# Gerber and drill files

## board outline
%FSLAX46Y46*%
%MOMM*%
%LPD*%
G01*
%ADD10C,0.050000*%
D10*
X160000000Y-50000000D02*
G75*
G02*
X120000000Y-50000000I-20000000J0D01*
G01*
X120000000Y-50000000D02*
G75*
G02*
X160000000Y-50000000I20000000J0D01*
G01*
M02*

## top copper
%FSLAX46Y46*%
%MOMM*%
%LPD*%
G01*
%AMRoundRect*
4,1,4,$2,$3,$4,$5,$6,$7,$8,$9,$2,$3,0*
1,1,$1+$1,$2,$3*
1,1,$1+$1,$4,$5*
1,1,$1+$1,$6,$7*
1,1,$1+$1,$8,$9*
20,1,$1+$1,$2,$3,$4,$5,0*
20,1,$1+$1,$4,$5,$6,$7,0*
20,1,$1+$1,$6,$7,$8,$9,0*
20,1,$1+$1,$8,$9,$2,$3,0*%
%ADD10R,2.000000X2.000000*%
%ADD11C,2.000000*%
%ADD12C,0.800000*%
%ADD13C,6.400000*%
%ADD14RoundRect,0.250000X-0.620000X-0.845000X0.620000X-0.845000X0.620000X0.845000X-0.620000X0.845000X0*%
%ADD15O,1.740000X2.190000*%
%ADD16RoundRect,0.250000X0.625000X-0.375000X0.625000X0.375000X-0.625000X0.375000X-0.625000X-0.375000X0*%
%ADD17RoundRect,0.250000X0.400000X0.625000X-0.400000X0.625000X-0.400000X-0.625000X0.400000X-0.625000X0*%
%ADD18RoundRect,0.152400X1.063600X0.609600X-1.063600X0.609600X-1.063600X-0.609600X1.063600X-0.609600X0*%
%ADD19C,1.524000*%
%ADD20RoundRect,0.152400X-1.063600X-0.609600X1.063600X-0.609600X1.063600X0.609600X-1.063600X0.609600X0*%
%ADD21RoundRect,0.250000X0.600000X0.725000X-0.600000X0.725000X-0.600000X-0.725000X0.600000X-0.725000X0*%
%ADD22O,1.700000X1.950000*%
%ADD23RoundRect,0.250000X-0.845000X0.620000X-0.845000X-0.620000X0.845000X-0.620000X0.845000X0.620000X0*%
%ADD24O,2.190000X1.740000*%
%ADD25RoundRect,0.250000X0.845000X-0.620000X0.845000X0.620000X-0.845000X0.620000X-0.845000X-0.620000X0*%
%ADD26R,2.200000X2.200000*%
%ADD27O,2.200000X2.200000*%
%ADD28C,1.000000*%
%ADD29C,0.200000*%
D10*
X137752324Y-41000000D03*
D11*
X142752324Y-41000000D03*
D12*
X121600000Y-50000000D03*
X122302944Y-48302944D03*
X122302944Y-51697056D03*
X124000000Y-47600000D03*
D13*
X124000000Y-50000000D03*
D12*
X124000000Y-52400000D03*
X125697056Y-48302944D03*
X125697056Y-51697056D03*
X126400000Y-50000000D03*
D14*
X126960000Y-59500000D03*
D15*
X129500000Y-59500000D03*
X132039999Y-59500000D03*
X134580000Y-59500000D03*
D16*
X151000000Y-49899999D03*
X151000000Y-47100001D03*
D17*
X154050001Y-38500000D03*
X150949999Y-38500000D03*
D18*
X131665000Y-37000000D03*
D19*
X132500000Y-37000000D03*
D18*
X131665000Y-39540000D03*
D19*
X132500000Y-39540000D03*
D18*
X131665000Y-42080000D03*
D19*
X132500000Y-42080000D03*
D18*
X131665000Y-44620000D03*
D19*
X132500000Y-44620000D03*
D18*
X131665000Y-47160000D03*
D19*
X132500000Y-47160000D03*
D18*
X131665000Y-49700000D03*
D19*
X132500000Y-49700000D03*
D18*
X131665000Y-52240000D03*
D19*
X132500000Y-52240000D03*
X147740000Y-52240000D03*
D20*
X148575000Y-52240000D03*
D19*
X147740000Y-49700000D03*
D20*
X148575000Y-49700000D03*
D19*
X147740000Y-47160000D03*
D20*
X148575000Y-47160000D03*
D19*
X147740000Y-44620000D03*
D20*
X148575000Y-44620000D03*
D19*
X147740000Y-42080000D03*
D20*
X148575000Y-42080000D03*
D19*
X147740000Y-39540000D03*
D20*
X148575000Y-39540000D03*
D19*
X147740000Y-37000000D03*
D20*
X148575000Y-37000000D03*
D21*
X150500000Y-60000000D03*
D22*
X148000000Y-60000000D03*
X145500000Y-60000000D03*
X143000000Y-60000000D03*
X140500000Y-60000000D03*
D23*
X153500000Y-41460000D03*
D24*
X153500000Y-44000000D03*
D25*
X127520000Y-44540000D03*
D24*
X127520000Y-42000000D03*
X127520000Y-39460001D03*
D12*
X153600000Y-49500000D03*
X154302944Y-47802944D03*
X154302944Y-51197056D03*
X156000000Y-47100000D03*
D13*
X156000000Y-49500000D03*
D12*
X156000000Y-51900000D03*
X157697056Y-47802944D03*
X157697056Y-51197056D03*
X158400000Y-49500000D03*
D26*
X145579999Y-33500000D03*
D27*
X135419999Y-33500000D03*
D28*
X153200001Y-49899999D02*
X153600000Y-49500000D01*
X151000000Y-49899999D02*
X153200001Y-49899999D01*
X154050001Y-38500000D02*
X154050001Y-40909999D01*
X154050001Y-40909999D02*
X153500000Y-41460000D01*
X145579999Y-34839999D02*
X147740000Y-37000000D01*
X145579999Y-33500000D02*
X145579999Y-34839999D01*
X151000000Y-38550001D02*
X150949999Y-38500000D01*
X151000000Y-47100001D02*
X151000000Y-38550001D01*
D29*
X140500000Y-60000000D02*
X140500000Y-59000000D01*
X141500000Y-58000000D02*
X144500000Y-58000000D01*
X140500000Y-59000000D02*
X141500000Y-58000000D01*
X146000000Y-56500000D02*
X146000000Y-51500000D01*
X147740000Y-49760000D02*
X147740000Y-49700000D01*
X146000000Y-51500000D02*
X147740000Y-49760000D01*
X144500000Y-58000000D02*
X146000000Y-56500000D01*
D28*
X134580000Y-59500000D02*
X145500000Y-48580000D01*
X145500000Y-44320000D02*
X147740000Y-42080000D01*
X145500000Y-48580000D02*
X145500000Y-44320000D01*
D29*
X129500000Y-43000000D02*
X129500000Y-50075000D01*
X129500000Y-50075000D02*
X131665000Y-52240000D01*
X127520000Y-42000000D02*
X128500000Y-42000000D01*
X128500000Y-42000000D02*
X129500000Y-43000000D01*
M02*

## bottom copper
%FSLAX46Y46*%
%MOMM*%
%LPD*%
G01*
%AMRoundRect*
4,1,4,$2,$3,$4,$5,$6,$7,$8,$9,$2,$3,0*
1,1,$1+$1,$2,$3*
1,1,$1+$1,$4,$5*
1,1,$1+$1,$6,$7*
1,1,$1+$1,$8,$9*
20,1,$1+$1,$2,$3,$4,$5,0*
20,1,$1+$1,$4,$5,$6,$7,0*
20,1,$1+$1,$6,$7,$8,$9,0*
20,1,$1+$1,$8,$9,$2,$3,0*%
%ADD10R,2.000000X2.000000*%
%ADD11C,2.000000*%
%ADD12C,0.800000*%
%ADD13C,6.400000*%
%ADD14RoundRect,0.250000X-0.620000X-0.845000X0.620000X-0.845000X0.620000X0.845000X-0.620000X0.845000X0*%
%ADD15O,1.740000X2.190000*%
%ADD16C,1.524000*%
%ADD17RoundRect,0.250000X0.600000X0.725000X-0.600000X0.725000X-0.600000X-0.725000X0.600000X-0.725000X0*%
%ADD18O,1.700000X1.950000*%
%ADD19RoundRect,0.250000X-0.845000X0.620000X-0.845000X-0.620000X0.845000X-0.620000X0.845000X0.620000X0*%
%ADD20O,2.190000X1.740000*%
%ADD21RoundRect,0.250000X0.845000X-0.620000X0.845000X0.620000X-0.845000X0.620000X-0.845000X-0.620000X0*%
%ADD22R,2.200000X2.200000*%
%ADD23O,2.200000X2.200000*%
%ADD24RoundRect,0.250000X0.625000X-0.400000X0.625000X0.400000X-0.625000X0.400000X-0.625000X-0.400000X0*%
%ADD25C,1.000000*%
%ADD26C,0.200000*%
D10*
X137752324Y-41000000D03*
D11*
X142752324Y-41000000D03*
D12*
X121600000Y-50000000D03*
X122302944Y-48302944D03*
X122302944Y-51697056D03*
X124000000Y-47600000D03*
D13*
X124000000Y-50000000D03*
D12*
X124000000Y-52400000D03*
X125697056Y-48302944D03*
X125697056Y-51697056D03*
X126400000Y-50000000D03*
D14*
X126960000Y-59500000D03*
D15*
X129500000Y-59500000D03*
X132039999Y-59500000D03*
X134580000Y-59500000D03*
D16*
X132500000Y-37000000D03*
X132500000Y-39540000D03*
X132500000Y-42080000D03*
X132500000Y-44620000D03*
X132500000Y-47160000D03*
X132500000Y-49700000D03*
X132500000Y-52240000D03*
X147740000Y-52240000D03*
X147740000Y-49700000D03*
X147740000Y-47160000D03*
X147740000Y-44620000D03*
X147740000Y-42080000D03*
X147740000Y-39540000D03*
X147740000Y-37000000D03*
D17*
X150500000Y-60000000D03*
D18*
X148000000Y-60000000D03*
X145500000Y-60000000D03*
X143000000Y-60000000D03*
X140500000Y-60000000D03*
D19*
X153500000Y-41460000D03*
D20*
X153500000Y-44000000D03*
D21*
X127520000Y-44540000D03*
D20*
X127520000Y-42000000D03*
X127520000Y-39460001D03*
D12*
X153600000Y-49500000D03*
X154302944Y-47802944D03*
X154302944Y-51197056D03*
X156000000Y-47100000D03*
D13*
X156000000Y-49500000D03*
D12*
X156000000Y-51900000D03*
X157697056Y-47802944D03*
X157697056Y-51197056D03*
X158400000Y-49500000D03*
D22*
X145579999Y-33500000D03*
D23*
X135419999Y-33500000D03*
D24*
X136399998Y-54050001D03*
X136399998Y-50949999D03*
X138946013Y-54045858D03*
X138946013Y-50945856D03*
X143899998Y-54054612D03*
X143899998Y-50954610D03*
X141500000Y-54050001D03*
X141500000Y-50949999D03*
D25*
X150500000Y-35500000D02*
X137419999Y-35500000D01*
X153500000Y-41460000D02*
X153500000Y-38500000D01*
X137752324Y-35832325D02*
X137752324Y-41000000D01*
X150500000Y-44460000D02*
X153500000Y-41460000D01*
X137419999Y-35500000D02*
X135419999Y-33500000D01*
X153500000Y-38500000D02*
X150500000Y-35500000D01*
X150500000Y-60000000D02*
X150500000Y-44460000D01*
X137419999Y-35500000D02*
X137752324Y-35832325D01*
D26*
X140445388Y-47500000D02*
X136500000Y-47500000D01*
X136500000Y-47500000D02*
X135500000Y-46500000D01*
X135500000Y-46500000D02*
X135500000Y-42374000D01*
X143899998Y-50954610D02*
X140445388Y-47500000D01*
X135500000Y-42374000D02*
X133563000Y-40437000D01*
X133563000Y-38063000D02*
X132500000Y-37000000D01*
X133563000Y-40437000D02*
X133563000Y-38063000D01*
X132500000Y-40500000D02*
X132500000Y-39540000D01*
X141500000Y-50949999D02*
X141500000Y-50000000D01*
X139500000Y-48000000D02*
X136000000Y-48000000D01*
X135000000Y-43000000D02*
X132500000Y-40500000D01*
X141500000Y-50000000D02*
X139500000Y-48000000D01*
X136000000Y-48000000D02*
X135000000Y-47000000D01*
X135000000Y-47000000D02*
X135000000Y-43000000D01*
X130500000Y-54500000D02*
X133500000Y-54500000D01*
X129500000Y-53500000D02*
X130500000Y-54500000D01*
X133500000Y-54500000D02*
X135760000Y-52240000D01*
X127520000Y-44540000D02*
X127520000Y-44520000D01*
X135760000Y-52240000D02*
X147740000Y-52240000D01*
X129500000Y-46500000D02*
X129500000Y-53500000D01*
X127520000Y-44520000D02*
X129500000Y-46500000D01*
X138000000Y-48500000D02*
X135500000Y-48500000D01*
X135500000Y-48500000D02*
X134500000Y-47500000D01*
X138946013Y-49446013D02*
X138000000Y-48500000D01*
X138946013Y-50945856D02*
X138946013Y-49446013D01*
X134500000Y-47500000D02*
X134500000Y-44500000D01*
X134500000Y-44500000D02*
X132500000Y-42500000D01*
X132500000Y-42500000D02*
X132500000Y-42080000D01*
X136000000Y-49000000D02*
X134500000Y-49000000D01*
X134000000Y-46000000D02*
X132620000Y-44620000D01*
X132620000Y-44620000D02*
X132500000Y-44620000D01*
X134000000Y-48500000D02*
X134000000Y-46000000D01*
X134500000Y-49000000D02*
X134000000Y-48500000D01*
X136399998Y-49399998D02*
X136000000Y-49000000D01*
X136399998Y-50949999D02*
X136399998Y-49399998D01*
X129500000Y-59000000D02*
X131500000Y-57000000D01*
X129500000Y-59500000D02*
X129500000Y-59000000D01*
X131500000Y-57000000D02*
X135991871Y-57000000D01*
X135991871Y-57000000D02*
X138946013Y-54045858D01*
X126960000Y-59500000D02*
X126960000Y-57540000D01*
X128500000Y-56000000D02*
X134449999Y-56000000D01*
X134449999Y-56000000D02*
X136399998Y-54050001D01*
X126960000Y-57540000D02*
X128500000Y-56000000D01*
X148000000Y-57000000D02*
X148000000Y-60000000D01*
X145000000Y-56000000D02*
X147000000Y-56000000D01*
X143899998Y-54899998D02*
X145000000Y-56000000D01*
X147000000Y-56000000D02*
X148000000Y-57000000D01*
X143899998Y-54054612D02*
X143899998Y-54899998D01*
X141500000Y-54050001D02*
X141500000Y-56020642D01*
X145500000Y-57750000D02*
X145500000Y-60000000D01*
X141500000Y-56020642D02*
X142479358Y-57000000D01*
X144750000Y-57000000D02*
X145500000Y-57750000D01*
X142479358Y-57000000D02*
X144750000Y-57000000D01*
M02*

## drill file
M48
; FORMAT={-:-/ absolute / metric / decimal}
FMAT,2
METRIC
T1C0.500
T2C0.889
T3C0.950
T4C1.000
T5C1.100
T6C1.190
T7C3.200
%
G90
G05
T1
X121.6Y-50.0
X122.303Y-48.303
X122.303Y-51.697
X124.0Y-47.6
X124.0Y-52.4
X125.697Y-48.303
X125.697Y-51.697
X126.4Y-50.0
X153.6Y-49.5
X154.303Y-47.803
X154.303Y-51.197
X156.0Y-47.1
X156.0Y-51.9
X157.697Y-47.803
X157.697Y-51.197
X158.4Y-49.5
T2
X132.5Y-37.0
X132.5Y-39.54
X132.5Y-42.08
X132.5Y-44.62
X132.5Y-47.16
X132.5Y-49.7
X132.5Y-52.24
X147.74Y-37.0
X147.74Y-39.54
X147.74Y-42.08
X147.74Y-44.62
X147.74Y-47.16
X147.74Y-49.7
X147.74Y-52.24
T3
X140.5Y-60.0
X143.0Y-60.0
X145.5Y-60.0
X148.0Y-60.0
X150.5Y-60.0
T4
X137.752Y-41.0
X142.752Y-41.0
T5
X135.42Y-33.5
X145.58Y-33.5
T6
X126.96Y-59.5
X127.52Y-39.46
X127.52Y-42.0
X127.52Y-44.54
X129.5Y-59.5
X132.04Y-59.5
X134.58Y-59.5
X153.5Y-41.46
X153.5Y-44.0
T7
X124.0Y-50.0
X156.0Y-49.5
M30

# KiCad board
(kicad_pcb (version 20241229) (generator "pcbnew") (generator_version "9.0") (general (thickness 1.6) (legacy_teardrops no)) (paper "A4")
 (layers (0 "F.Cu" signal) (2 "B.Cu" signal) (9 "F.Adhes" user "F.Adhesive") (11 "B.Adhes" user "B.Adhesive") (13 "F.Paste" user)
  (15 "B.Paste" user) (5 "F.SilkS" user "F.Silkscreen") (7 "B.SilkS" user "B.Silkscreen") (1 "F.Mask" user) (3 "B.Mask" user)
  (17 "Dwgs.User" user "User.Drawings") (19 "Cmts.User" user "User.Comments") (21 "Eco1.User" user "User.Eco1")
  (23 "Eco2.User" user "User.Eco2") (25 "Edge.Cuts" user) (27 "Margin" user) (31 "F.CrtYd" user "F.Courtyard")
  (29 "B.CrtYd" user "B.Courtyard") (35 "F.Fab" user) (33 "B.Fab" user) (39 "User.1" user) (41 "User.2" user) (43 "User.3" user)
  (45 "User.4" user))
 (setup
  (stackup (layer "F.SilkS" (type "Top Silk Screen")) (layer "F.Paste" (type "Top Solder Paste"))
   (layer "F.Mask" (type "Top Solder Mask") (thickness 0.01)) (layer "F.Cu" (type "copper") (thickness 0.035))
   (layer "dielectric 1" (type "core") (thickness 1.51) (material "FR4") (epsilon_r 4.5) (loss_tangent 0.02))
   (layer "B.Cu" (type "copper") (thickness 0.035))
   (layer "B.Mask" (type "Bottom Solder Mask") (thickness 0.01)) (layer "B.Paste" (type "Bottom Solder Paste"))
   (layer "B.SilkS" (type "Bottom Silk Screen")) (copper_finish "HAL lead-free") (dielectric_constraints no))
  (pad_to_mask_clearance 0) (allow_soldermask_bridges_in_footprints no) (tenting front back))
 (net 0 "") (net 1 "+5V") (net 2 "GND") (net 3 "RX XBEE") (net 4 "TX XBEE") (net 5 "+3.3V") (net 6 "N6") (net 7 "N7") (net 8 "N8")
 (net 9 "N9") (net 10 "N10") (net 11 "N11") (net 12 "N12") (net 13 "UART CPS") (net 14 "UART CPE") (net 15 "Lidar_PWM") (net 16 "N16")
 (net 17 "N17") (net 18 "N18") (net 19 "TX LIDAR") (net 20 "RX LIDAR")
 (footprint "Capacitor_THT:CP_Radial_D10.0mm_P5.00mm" (layer "F.Cu") (at 137.752324 41)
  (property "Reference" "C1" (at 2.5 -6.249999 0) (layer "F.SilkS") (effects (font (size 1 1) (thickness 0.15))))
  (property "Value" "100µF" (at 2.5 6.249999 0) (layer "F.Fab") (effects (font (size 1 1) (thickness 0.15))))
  (pad "1" thru_hole rect (at 0 0) (size 2 2) (drill 1) (layers "*.Cu" "*.Mask") (remove_unused_layers no) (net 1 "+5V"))
  (pad "2" thru_hole circle (at 5 0) (size 2 2) (drill 1) (layers "*.Cu" "*.Mask") (remove_unused_layers no) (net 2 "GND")))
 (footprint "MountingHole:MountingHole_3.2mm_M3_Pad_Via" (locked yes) (layer "F.Cu") (at 124 50)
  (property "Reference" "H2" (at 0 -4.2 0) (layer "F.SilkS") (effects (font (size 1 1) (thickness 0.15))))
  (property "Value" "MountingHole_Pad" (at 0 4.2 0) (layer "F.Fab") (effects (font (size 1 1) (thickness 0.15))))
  (pad "1" thru_hole circle (at -2.4 0) (size 0.8 0.8) (drill 0.5) (layers "*.Cu" "*.Mask") (remove_unused_layers no) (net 2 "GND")
   (zone_connect 2))
  (pad "1" thru_hole circle (at -1.697056 -1.697056) (size 0.8 0.8) (drill 0.5) (layers "*.Cu" "*.Mask") (remove_unused_layers no)
   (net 2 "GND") (zone_connect 2))
  (pad "1" thru_hole circle (at -1.697056 1.697056) (size 0.8 0.8) (drill 0.5) (layers "*.Cu" "*.Mask") (remove_unused_layers no)
   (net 2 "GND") (zone_connect 2))
  (pad "1" thru_hole circle (at 0 -2.4) (size 0.8 0.8) (drill 0.5) (layers "*.Cu" "*.Mask") (remove_unused_layers no) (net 2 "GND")
   (zone_connect 2))
  (pad "1" thru_hole circle (at 0 0) (size 6.4 6.4) (drill 3.2) (layers "*.Cu" "*.Mask") (remove_unused_layers no) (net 2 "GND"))
  (pad "1" thru_hole circle (at 0 2.4) (size 0.8 0.8) (drill 0.5) (layers "*.Cu" "*.Mask") (remove_unused_layers no) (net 2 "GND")
   (zone_connect 2))
  (pad "1" thru_hole circle (at 1.697056 -1.697056) (size 0.8 0.8) (drill 0.5) (layers "*.Cu" "*.Mask") (remove_unused_layers no)
   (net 2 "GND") (zone_connect 2))
  (pad "1" thru_hole circle (at 1.697056 1.697056) (size 0.8 0.8) (drill 0.5) (layers "*.Cu" "*.Mask") (remove_unused_layers no)
   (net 2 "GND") (zone_connect 2))
  (pad "1" thru_hole circle (at 2.4 0) (size 0.8 0.8) (drill 0.5) (layers "*.Cu" "*.Mask") (remove_unused_layers no) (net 2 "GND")
   (zone_connect 2)))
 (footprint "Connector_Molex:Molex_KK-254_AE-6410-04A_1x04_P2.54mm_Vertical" (layer "F.Cu") (at 126.96 59.5)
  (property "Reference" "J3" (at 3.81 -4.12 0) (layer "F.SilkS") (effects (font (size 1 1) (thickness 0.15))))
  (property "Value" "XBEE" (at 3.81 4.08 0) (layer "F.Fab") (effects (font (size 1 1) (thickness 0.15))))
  (pad "1" thru_hole roundrect (at 0 0) (size 1.74 2.19) (drill 1.19) (layers "*.Cu" "*.Mask") (remove_unused_layers no)
   (roundrect_rratio 0.143678) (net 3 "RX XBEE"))
  (pad "2" thru_hole oval (at 2.54 0) (size 1.74 2.19) (drill 1.19) (layers "*.Cu" "*.Mask") (remove_unused_layers no) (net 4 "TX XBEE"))
  (pad "3" thru_hole oval (at 5.079999 0) (size 1.74 2.19) (drill 1.19) (layers "*.Cu" "*.Mask") (remove_unused_layers no) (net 2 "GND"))
  (pad "4" thru_hole oval (at 7.62 0) (size 1.74 2.19) (drill 1.19) (layers "*.Cu" "*.Mask") (remove_unused_layers no) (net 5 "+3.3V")))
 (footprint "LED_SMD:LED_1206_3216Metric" (layer "F.Cu") (at 151 48.5 90)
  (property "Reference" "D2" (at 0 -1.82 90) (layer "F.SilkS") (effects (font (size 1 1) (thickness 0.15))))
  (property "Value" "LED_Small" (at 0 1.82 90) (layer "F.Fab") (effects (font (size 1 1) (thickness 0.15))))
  (pad "1" smd roundrect (at -1.399999 0 90) (size 1.25 1.75) (layers "F.Cu" "F.Mask" "F.Paste") (roundrect_rratio 0.2) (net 2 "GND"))
  (pad "2" smd roundrect (at 1.399999 0 90) (size 1.25 1.75) (layers "F.Cu" "F.Mask" "F.Paste") (roundrect_rratio 0.2) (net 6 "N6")))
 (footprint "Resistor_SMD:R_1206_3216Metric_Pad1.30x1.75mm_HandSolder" (layer "F.Cu") (at 152.5 38.5 180)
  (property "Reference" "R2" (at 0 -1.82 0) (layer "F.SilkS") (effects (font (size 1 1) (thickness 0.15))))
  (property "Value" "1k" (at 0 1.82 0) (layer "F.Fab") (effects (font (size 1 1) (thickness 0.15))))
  (pad "1" smd roundrect (at -1.550001 0 180) (size 1.3 1.75) (layers "F.Cu" "F.Mask" "F.Paste") (roundrect_rratio 0.192308) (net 1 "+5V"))
  (pad "2" smd roundrect (at 1.550001 0 180) (size 1.3 1.75) (layers "F.Cu" "F.Mask" "F.Paste") (roundrect_rratio 0.192308) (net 6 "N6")))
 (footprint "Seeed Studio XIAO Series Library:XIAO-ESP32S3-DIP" (layer "F.Cu") (at 140.12 44.62)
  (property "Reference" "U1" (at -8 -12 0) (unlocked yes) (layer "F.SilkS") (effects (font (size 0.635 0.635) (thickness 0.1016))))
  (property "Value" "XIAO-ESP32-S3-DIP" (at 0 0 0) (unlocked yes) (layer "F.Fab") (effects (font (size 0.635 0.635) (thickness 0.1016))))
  (pad "1" smd roundrect (at -8.455 -7.62 180) (size 2.432 1.524) (layers "F.Cu" "F.Mask") (roundrect_rratio 0.1) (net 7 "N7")
   (thermal_bridge_angle 45))
  (pad "1" thru_hole circle (at -7.62 -7.62 180) (size 1.524 1.524) (drill 0.889) (layers "*.Cu" "*.Mask") (remove_unused_layers no)
   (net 7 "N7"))
  (pad "2" smd roundrect (at -8.455 -5.08 180) (size 2.432 1.524) (layers "F.Cu" "F.Mask") (roundrect_rratio 0.1) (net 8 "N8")
   (thermal_bridge_angle 45))
  (pad "2" thru_hole circle (at -7.62 -5.08 180) (size 1.524 1.524) (drill 0.889) (layers "*.Cu" "*.Mask") (remove_unused_layers no)
   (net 8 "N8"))
  (pad "3" smd roundrect (at -8.455 -2.54 180) (size 2.432 1.524) (layers "F.Cu" "F.Mask") (roundrect_rratio 0.1) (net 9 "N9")
   (thermal_bridge_angle 45))
  (pad "3" thru_hole circle (at -7.62 -2.54 180) (size 1.524 1.524) (drill 0.889) (layers "*.Cu" "*.Mask") (remove_unused_layers no)
   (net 9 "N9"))
  (pad "4" smd roundrect (at -8.455 0 180) (size 2.432 1.524) (layers "F.Cu" "F.Mask") (roundrect_rratio 0.1) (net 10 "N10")
   (thermal_bridge_angle 45))
  (pad "4" thru_hole circle (at -7.62 0 180) (size 1.524 1.524) (drill 0.889) (layers "*.Cu" "*.Mask") (remove_unused_layers no)
   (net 10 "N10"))
  (pad "5" smd roundrect (at -8.455 2.54 180) (size 2.432 1.524) (layers "F.Cu" "F.Mask") (roundrect_rratio 0.1) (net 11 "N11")
   (thermal_bridge_angle 45))
  (pad "5" thru_hole circle (at -7.62 2.54 180) (size 1.524 1.524) (drill 0.889) (layers "*.Cu" "*.Mask") (remove_unused_layers no)
   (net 11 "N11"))
  (pad "6" smd roundrect (at -8.455 5.08 180) (size 2.432 1.524) (layers "F.Cu" "F.Mask") (roundrect_rratio 0.1) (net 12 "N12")
   (thermal_bridge_angle 45))
  (pad "6" thru_hole circle (at -7.62 5.08 180) (size 1.524 1.524) (drill 0.889) (layers "*.Cu" "*.Mask") (remove_unused_layers no)
   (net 12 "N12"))
  (pad "7" smd roundrect (at -8.455 7.62 180) (size 2.432 1.524) (layers "F.Cu" "F.Mask") (roundrect_rratio 0.1) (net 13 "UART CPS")
   (thermal_bridge_angle 45))
  (pad "7" thru_hole circle (at -7.62 7.62 180) (size 1.524 1.524) (drill 0.889) (layers "*.Cu" "*.Mask") (remove_unused_layers no)
   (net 13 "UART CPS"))
  (pad "8" thru_hole circle (at 7.62 7.62) (size 1.524 1.524) (drill 0.889) (layers "*.Cu" "*.Mask") (remove_unused_layers no)
   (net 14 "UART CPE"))
  (pad "8" smd roundrect (at 8.455 7.62) (size 2.432 1.524) (layers "F.Cu" "F.Mask") (roundrect_rratio 0.1) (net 14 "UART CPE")
   (thermal_bridge_angle 45))
  (pad "9" thru_hole circle (at 7.62 5.08) (size 1.524 1.524) (drill 0.889) (layers "*.Cu" "*.Mask") (remove_unused_layers no)
   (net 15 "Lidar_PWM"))
  (pad "9" smd roundrect (at 8.455 5.08) (size 2.432 1.524) (layers "F.Cu" "F.Mask") (roundrect_rratio 0.1) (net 15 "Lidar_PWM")
   (thermal_bridge_angle 45))
  (pad "10" thru_hole circle (at 7.62 2.54) (size 1.524 1.524) (drill 0.889) (layers "*.Cu" "*.Mask") (remove_unused_layers no)
   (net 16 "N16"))
  (pad "10" smd roundrect (at 8.455 2.54) (size 2.432 1.524) (layers "F.Cu" "F.Mask") (roundrect_rratio 0.1) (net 16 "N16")
   (thermal_bridge_angle 45))
  (pad "11" thru_hole circle (at 7.62 0) (size 1.524 1.524) (drill 0.889) (layers "*.Cu" "*.Mask") (remove_unused_layers no) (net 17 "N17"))
  (pad "11" smd roundrect (at 8.455 0) (size 2.432 1.524) (layers "F.Cu" "F.Mask") (roundrect_rratio 0.1) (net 17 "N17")
   (thermal_bridge_angle 45))
  (pad "12" thru_hole circle (at 7.62 -2.54) (size 1.524 1.524) (drill 0.889) (layers "*.Cu" "*.Mask") (remove_unused_layers no)
   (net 5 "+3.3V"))
  (pad "12" smd roundrect (at 8.455 -2.54) (size 2.432 1.524) (layers "F.Cu" "F.Mask") (roundrect_rratio 0.1) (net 5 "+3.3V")
   (thermal_bridge_angle 45))
  (pad "13" thru_hole circle (at 7.62 -5.08) (size 1.524 1.524) (drill 0.889) (layers "*.Cu" "*.Mask") (remove_unused_layers no)
   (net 2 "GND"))
  (pad "13" smd roundrect (at 8.455 -5.08) (size 2.432 1.524) (layers "F.Cu" "F.Mask") (roundrect_rratio 0.1) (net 2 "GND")
   (thermal_bridge_angle 45))
  (pad "14" thru_hole circle (at 7.62 -7.62) (size 1.524 1.524) (drill 0.889) (layers "*.Cu" "*.Mask") (remove_unused_layers no)
   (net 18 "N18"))
  (pad "14" smd roundrect (at 8.455 -7.62) (size 2.432 1.524) (layers "F.Cu" "F.Mask") (roundrect_rratio 0.1) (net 18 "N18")
   (thermal_bridge_angle 45)))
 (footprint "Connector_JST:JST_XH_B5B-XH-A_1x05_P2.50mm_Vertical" (layer "F.Cu") (at 150.5 60 180)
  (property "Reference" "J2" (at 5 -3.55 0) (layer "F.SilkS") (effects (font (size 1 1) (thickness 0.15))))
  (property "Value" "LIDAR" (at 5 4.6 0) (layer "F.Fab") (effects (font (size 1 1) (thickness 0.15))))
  (pad "1" thru_hole roundrect (at 0 0 180) (size 1.7 1.95) (drill 0.95) (layers "*.Cu" "*.Mask") (remove_unused_layers no)
   (roundrect_rratio 0.147059) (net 1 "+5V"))
  (pad "2" thru_hole oval (at 2.5 0 180) (size 1.7 1.95) (drill 0.95) (layers "*.Cu" "*.Mask") (remove_unused_layers no) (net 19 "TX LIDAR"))
  (pad "3" thru_hole oval (at 5 0 180) (size 1.7 1.95) (drill 0.95) (layers "*.Cu" "*.Mask") (remove_unused_layers no) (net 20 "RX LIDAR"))
  (pad "4" thru_hole oval (at 7.5 0 180) (size 1.7 1.95) (drill 0.95) (layers "*.Cu" "*.Mask") (remove_unused_layers no) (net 2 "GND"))
  (pad "5" thru_hole oval (at 10 0 180) (size 1.7 1.95) (drill 0.95) (layers "*.Cu" "*.Mask") (remove_unused_layers no) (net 15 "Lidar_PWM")))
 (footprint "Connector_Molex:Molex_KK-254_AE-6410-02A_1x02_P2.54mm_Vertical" (layer "F.Cu") (at 153.5 41.46 -90)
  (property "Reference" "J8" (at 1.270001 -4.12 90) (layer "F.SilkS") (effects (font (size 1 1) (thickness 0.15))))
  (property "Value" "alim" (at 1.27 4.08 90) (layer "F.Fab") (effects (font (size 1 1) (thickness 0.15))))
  (pad "1" thru_hole roundrect (at 0 0 270) (size 1.74 2.19) (drill 1.19) (layers "*.Cu" "*.Mask") (remove_unused_layers no)
   (roundrect_rratio 0.143678) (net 1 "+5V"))
  (pad "2" thru_hole oval (at 2.54 0 270) (size 1.74 2.19) (drill 1.19) (layers "*.Cu" "*.Mask") (remove_unused_layers no) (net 2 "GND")))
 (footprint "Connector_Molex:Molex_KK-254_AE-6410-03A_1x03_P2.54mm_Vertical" (layer "F.Cu") (at 127.52 44.54 90)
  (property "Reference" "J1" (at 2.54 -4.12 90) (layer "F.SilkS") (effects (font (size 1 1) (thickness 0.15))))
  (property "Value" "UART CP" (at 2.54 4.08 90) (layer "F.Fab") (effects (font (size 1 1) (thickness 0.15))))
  (pad "1" thru_hole roundrect (at 0 0 90) (size 1.74 2.19) (drill 1.19) (layers "*.Cu" "*.Mask") (remove_unused_layers no)
   (roundrect_rratio 0.143678) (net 14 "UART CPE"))
  (pad "2" thru_hole oval (at 2.54 0 90) (size 1.74 2.19) (drill 1.19) (layers "*.Cu" "*.Mask") (remove_unused_layers no)
   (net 13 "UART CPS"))
  (pad "3" thru_hole oval (at 5.079999 0 90) (size 1.74 2.19) (drill 1.19) (layers "*.Cu" "*.Mask") (remove_unused_layers no) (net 2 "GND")))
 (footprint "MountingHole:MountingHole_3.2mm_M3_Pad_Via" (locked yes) (layer "F.Cu") (at 156 49.5)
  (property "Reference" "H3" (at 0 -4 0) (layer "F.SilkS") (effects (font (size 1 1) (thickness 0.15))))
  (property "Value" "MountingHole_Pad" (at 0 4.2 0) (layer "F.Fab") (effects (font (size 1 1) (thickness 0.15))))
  (pad "1" thru_hole circle (at -2.4 0) (size 0.8 0.8) (drill 0.5) (layers "*.Cu" "*.Mask") (remove_unused_layers no) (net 2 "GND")
   (zone_connect 2))
  (pad "1" thru_hole circle (at -1.697056 -1.697056) (size 0.8 0.8) (drill 0.5) (layers "*.Cu" "*.Mask") (remove_unused_layers no)
   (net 2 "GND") (zone_connect 2))
  (pad "1" thru_hole circle (at -1.697056 1.697056) (size 0.8 0.8) (drill 0.5) (layers "*.Cu" "*.Mask") (remove_unused_layers no)
   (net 2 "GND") (zone_connect 2))
  (pad "1" thru_hole circle (at 0 -2.4) (size 0.8 0.8) (drill 0.5) (layers "*.Cu" "*.Mask") (remove_unused_layers no) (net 2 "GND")
   (zone_connect 2))
  (pad "1" thru_hole circle (at 0 0) (size 6.4 6.4) (drill 3.2) (layers "*.Cu" "*.Mask") (remove_unused_layers no) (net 2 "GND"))
  (pad "1" thru_hole circle (at 0 2.4) (size 0.8 0.8) (drill 0.5) (layers "*.Cu" "*.Mask") (remove_unused_layers no) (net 2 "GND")
   (zone_connect 2))
  (pad "1" thru_hole circle (at 1.697056 -1.697056) (size 0.8 0.8) (drill 0.5) (layers "*.Cu" "*.Mask") (remove_unused_layers no)
   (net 2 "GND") (zone_connect 2))
  (pad "1" thru_hole circle (at 1.697056 1.697056) (size 0.8 0.8) (drill 0.5) (layers "*.Cu" "*.Mask") (remove_unused_layers no)
   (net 2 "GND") (zone_connect 2))
  (pad "1" thru_hole circle (at 2.4 0) (size 0.8 0.8) (drill 0.5) (layers "*.Cu" "*.Mask") (remove_unused_layers no) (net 2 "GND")
   (zone_connect 2)))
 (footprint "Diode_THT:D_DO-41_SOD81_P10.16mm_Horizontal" (layer "F.Cu") (at 145.579999 33.5 180)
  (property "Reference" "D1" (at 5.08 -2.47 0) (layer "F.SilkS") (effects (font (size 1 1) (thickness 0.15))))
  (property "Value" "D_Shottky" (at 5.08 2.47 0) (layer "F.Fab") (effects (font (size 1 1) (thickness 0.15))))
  (pad "1" thru_hole rect (at 0 0 180) (size 2.2 2.2) (drill 1.1) (layers "*.Cu" "*.Mask") (remove_unused_layers no) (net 18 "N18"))
  (pad "2" thru_hole oval (at 10.16 0 180) (size 2.2 2.2) (drill 1.1) (layers "*.Cu" "*.Mask") (remove_unused_layers no) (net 1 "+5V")))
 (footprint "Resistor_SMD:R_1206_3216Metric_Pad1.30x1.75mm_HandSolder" (layer "B.Cu") (at 136.399998 52.5 90)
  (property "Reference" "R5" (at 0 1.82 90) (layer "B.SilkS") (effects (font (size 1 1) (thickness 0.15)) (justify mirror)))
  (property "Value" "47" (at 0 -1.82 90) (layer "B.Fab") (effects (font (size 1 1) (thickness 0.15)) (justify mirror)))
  (pad "1" smd roundrect (at -1.550001 0 90) (size 1.3 1.75) (layers "B.Cu" "B.Mask" "B.Paste") (roundrect_rratio 0.192308)
   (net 3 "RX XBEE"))
  (pad "2" smd roundrect (at 1.550001 0 90) (size 1.3 1.75) (layers "B.Cu" "B.Mask" "B.Paste") (roundrect_rratio 0.192308) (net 10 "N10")))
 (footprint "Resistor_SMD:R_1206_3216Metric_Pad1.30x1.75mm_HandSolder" (layer "B.Cu") (at 138.946013 52.495857 90)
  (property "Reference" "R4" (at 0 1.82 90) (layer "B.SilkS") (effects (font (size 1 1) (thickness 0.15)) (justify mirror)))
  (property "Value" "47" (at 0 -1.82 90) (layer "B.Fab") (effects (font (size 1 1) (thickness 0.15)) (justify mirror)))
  (pad "1" smd roundrect (at -1.550001 0 90) (size 1.3 1.75) (layers "B.Cu" "B.Mask" "B.Paste") (roundrect_rratio 0.192308)
   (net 4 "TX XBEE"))
  (pad "2" smd roundrect (at 1.550001 0 90) (size 1.3 1.75) (layers "B.Cu" "B.Mask" "B.Paste") (roundrect_rratio 0.192308) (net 9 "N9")))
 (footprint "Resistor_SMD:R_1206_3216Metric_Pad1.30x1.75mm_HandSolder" (layer "B.Cu") (at 143.899998 52.504611 90)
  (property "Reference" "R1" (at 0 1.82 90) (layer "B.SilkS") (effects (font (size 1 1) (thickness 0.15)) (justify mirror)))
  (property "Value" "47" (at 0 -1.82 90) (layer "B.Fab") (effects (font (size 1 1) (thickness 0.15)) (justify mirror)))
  (pad "1" smd roundrect (at -1.550001 0 90) (size 1.3 1.75) (layers "B.Cu" "B.Mask" "B.Paste") (roundrect_rratio 0.192308)
   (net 19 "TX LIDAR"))
  (pad "2" smd roundrect (at 1.550001 0 90) (size 1.3 1.75) (layers "B.Cu" "B.Mask" "B.Paste") (roundrect_rratio 0.192308) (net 7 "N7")))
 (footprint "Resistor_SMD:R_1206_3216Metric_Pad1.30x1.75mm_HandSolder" (layer "B.Cu") (at 141.5 52.5 90)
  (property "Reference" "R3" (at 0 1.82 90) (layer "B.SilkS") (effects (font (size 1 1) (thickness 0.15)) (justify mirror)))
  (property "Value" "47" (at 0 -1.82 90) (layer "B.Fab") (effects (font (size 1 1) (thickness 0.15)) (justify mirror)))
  (pad "1" smd roundrect (at -1.550001 0 90) (size 1.3 1.75) (layers "B.Cu" "B.Mask" "B.Paste") (roundrect_rratio 0.192308)
   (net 20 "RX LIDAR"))
  (pad "2" smd roundrect (at 1.550001 0 90) (size 1.3 1.75) (layers "B.Cu" "B.Mask" "B.Paste") (roundrect_rratio 0.192308) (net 8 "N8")))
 (gr_circle (center 140 50) (end 140 70) (stroke (width 0.05) (type default)) (fill no) (layer "Edge.Cuts"))
 (segment (start 153.200001 49.899999) (end 153.6 49.5) (width 1) (layer "F.Cu") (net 2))
 (segment (start 151 49.899999) (end 153.200001 49.899999) (width 1) (layer "F.Cu") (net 2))
 (segment (start 154.050001 38.5) (end 154.050001 40.909999) (width 1) (layer "F.Cu") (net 1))
 (segment (start 154.050001 40.909999) (end 153.5 41.46) (width 1) (layer "F.Cu") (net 1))
 (segment (start 150.5 35.5) (end 137.419999 35.5) (width 1) (layer "B.Cu") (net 1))
 (segment (start 153.5 41.46) (end 153.5 38.5) (width 1) (layer "B.Cu") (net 1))
 (segment (start 137.752324 35.832325) (end 137.752324 41) (width 1) (layer "B.Cu") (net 1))
 (segment (start 150.5 44.46) (end 153.5 41.46) (width 1) (layer "B.Cu") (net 1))
 (segment (start 137.419999 35.5) (end 135.419999 33.5) (width 1) (layer "B.Cu") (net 1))
 (segment (start 153.5 38.5) (end 150.5 35.5) (width 1) (layer "B.Cu") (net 1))
 (segment (start 150.5 60) (end 150.5 44.46) (width 1) (layer "B.Cu") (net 1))
 (segment (start 137.419999 35.5) (end 137.752324 35.832325) (width 1) (layer "B.Cu") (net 1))
 (segment (start 145.579999 34.839999) (end 147.74 37) (width 1) (layer "F.Cu") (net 18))
 (segment (start 145.579999 33.5) (end 145.579999 34.839999) (width 1) (layer "F.Cu") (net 18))
 (segment (start 151 38.550001) (end 150.949999 38.5) (width 1) (layer "F.Cu") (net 6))
 (segment (start 151 47.100001) (end 151 38.550001) (width 1) (layer "F.Cu") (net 6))
 (segment (start 140.5 60) (end 140.5 59) (width 0.2) (layer "F.Cu") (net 15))
 (segment (start 141.5 58) (end 144.5 58) (width 0.2) (layer "F.Cu") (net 15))
 (segment (start 140.5 59) (end 141.5 58) (width 0.2) (layer "F.Cu") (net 15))
 (segment (start 146 56.5) (end 146 51.5) (width 0.2) (layer "F.Cu") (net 15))
 (segment (start 147.74 49.76) (end 147.74 49.7) (width 0.2) (layer "F.Cu") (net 15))
 (segment (start 146 51.5) (end 147.74 49.76) (width 0.2) (layer "F.Cu") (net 15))
 (segment (start 144.5 58) (end 146 56.5) (width 0.2) (layer "F.Cu") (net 15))
 (segment (start 134.58 59.5) (end 145.5 48.58) (width 1) (layer "F.Cu") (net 5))
 (segment (start 145.5 44.32) (end 147.74 42.08) (width 1) (layer "F.Cu") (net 5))
 (segment (start 145.5 48.58) (end 145.5 44.32) (width 1) (layer "F.Cu") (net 5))
 (segment (start 140.445388 47.5) (end 136.5 47.5) (width 0.2) (layer "B.Cu") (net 7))
 (segment (start 136.5 47.5) (end 135.5 46.5) (width 0.2) (layer "B.Cu") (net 7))
 (segment (start 135.5 46.5) (end 135.5 42.374) (width 0.2) (layer "B.Cu") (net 7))
 (segment (start 143.899998 50.95461) (end 140.445388 47.5) (width 0.2) (layer "B.Cu") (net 7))
 (segment (start 135.5 42.374) (end 133.563 40.437) (width 0.2) (layer "B.Cu") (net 7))
 (segment (start 133.563 38.063) (end 132.5 37) (width 0.2) (layer "B.Cu") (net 7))
 (segment (start 133.563 40.437) (end 133.563 38.063) (width 0.2) (layer "B.Cu") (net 7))
 (segment (start 132.5 40.5) (end 132.5 39.54) (width 0.2) (layer "B.Cu") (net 8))
 (segment (start 141.5 50.949999) (end 141.5 50) (width 0.2) (layer "B.Cu") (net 8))
 (segment (start 139.5 48) (end 136 48) (width 0.2) (layer "B.Cu") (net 8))
 (segment (start 135 43) (end 132.5 40.5) (width 0.2) (layer "B.Cu") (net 8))
 (segment (start 141.5 50) (end 139.5 48) (width 0.2) (layer "B.Cu") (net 8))
 (segment (start 136 48) (end 135 47) (width 0.2) (layer "B.Cu") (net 8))
 (segment (start 135 47) (end 135 43) (width 0.2) (layer "B.Cu") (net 8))
 (segment (start 130.5 54.5) (end 133.5 54.5) (width 0.2) (layer "B.Cu") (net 14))
 (segment (start 129.5 53.5) (end 130.5 54.5) (width 0.2) (layer "B.Cu") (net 14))
 (segment (start 133.5 54.5) (end 135.76 52.24) (width 0.2) (layer "B.Cu") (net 14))
 (segment (start 127.52 44.54) (end 127.52 44.52) (width 0.2) (layer "B.Cu") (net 14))
 (segment (start 135.76 52.24) (end 147.74 52.24) (width 0.2) (layer "B.Cu") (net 14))
 (segment (start 129.5 46.5) (end 129.5 53.5) (width 0.2) (layer "B.Cu") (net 14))
 (segment (start 127.52 44.52) (end 129.5 46.5) (width 0.2) (layer "B.Cu") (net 14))
 (segment (start 138 48.5) (end 135.5 48.5) (width 0.2) (layer "B.Cu") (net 9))
 (segment (start 135.5 48.5) (end 134.5 47.5) (width 0.2) (layer "B.Cu") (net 9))
 (segment (start 138.946013 49.446013) (end 138 48.5) (width 0.2) (layer "B.Cu") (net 9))
 (segment (start 138.946013 50.945856) (end 138.946013 49.446013) (width 0.2) (layer "B.Cu") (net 9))
 (segment (start 134.5 47.5) (end 134.5 44.5) (width 0.2) (layer "B.Cu") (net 9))
 (segment (start 134.5 44.5) (end 132.5 42.5) (width 0.2) (layer "B.Cu") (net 9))
 (segment (start 132.5 42.5) (end 132.5 42.08) (width 0.2) (layer "B.Cu") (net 9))
 (segment (start 129.5 43) (end 129.5 50.075) (width 0.2) (layer "F.Cu") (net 13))
 (segment (start 129.5 50.075) (end 131.665 52.24) (width 0.2) (layer "F.Cu") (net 13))
 (segment (start 127.52 42) (end 128.5 42) (width 0.2) (layer "F.Cu") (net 13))
 (segment (start 128.5 42) (end 129.5 43) (width 0.2) (layer "F.Cu") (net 13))
 (segment (start 136 49) (end 134.5 49) (width 0.2) (layer "B.Cu") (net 10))
 (segment (start 134 46) (end 132.62 44.62) (width 0.2) (layer "B.Cu") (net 10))
 (segment (start 132.62 44.62) (end 132.5 44.62) (width 0.2) (layer "B.Cu") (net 10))
 (segment (start 134 48.5) (end 134 46) (width 0.2) (layer "B.Cu") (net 10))
 (segment (start 134.5 49) (end 134 48.5) (width 0.2) (layer "B.Cu") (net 10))
 (segment (start 136.399998 49.399998) (end 136 49) (width 0.2) (layer "B.Cu") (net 10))
 (segment (start 136.399998 50.949999) (end 136.399998 49.399998) (width 0.2) (layer "B.Cu") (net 10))
 (segment (start 129.5 59) (end 131.5 57) (width 0.2) (layer "B.Cu") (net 4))
 (segment (start 129.5 59.5) (end 129.5 59) (width 0.2) (layer "B.Cu") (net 4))
 (segment (start 131.5 57) (end 135.991871 57) (width 0.2) (layer "B.Cu") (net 4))
 (segment (start 135.991871 57) (end 138.946013 54.045858) (width 0.2) (layer "B.Cu") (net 4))
 (segment (start 126.96 59.5) (end 126.96 57.54) (width 0.2) (layer "B.Cu") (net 3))
 (segment (start 128.5 56) (end 134.449999 56) (width 0.2) (layer "B.Cu") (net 3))
 (segment (start 134.449999 56) (end 136.399998 54.050001) (width 0.2) (layer "B.Cu") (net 3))
 (segment (start 126.96 57.54) (end 128.5 56) (width 0.2) (layer "B.Cu") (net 3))
 (segment (start 148 57) (end 148 60) (width 0.2) (layer "B.Cu") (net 19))
 (segment (start 145 56) (end 147 56) (width 0.2) (layer "B.Cu") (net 19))
 (segment (start 143.899998 54.899998) (end 145 56) (width 0.2) (layer "B.Cu") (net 19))
 (segment (start 147 56) (end 148 57) (width 0.2) (layer "B.Cu") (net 19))
 (segment (start 143.899998 54.054612) (end 143.899998 54.899998) (width 0.2) (layer "B.Cu") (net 19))
 (segment (start 141.5 54.050001) (end 141.5 56.020642) (width 0.2) (layer "B.Cu") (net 20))
 (segment (start 145.5 57.75) (end 145.5 60) (width 0.2) (layer "B.Cu") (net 20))
 (segment (start 141.5 56.020642) (end 142.479358 57) (width 0.2) (layer "B.Cu") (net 20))
 (segment (start 144.75 57) (end 145.5 57.75) (width 0.2) (layer "B.Cu") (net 20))
 (segment (start 142.479358 57) (end 144.75 57) (width 0.2) (layer "B.Cu") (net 20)))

